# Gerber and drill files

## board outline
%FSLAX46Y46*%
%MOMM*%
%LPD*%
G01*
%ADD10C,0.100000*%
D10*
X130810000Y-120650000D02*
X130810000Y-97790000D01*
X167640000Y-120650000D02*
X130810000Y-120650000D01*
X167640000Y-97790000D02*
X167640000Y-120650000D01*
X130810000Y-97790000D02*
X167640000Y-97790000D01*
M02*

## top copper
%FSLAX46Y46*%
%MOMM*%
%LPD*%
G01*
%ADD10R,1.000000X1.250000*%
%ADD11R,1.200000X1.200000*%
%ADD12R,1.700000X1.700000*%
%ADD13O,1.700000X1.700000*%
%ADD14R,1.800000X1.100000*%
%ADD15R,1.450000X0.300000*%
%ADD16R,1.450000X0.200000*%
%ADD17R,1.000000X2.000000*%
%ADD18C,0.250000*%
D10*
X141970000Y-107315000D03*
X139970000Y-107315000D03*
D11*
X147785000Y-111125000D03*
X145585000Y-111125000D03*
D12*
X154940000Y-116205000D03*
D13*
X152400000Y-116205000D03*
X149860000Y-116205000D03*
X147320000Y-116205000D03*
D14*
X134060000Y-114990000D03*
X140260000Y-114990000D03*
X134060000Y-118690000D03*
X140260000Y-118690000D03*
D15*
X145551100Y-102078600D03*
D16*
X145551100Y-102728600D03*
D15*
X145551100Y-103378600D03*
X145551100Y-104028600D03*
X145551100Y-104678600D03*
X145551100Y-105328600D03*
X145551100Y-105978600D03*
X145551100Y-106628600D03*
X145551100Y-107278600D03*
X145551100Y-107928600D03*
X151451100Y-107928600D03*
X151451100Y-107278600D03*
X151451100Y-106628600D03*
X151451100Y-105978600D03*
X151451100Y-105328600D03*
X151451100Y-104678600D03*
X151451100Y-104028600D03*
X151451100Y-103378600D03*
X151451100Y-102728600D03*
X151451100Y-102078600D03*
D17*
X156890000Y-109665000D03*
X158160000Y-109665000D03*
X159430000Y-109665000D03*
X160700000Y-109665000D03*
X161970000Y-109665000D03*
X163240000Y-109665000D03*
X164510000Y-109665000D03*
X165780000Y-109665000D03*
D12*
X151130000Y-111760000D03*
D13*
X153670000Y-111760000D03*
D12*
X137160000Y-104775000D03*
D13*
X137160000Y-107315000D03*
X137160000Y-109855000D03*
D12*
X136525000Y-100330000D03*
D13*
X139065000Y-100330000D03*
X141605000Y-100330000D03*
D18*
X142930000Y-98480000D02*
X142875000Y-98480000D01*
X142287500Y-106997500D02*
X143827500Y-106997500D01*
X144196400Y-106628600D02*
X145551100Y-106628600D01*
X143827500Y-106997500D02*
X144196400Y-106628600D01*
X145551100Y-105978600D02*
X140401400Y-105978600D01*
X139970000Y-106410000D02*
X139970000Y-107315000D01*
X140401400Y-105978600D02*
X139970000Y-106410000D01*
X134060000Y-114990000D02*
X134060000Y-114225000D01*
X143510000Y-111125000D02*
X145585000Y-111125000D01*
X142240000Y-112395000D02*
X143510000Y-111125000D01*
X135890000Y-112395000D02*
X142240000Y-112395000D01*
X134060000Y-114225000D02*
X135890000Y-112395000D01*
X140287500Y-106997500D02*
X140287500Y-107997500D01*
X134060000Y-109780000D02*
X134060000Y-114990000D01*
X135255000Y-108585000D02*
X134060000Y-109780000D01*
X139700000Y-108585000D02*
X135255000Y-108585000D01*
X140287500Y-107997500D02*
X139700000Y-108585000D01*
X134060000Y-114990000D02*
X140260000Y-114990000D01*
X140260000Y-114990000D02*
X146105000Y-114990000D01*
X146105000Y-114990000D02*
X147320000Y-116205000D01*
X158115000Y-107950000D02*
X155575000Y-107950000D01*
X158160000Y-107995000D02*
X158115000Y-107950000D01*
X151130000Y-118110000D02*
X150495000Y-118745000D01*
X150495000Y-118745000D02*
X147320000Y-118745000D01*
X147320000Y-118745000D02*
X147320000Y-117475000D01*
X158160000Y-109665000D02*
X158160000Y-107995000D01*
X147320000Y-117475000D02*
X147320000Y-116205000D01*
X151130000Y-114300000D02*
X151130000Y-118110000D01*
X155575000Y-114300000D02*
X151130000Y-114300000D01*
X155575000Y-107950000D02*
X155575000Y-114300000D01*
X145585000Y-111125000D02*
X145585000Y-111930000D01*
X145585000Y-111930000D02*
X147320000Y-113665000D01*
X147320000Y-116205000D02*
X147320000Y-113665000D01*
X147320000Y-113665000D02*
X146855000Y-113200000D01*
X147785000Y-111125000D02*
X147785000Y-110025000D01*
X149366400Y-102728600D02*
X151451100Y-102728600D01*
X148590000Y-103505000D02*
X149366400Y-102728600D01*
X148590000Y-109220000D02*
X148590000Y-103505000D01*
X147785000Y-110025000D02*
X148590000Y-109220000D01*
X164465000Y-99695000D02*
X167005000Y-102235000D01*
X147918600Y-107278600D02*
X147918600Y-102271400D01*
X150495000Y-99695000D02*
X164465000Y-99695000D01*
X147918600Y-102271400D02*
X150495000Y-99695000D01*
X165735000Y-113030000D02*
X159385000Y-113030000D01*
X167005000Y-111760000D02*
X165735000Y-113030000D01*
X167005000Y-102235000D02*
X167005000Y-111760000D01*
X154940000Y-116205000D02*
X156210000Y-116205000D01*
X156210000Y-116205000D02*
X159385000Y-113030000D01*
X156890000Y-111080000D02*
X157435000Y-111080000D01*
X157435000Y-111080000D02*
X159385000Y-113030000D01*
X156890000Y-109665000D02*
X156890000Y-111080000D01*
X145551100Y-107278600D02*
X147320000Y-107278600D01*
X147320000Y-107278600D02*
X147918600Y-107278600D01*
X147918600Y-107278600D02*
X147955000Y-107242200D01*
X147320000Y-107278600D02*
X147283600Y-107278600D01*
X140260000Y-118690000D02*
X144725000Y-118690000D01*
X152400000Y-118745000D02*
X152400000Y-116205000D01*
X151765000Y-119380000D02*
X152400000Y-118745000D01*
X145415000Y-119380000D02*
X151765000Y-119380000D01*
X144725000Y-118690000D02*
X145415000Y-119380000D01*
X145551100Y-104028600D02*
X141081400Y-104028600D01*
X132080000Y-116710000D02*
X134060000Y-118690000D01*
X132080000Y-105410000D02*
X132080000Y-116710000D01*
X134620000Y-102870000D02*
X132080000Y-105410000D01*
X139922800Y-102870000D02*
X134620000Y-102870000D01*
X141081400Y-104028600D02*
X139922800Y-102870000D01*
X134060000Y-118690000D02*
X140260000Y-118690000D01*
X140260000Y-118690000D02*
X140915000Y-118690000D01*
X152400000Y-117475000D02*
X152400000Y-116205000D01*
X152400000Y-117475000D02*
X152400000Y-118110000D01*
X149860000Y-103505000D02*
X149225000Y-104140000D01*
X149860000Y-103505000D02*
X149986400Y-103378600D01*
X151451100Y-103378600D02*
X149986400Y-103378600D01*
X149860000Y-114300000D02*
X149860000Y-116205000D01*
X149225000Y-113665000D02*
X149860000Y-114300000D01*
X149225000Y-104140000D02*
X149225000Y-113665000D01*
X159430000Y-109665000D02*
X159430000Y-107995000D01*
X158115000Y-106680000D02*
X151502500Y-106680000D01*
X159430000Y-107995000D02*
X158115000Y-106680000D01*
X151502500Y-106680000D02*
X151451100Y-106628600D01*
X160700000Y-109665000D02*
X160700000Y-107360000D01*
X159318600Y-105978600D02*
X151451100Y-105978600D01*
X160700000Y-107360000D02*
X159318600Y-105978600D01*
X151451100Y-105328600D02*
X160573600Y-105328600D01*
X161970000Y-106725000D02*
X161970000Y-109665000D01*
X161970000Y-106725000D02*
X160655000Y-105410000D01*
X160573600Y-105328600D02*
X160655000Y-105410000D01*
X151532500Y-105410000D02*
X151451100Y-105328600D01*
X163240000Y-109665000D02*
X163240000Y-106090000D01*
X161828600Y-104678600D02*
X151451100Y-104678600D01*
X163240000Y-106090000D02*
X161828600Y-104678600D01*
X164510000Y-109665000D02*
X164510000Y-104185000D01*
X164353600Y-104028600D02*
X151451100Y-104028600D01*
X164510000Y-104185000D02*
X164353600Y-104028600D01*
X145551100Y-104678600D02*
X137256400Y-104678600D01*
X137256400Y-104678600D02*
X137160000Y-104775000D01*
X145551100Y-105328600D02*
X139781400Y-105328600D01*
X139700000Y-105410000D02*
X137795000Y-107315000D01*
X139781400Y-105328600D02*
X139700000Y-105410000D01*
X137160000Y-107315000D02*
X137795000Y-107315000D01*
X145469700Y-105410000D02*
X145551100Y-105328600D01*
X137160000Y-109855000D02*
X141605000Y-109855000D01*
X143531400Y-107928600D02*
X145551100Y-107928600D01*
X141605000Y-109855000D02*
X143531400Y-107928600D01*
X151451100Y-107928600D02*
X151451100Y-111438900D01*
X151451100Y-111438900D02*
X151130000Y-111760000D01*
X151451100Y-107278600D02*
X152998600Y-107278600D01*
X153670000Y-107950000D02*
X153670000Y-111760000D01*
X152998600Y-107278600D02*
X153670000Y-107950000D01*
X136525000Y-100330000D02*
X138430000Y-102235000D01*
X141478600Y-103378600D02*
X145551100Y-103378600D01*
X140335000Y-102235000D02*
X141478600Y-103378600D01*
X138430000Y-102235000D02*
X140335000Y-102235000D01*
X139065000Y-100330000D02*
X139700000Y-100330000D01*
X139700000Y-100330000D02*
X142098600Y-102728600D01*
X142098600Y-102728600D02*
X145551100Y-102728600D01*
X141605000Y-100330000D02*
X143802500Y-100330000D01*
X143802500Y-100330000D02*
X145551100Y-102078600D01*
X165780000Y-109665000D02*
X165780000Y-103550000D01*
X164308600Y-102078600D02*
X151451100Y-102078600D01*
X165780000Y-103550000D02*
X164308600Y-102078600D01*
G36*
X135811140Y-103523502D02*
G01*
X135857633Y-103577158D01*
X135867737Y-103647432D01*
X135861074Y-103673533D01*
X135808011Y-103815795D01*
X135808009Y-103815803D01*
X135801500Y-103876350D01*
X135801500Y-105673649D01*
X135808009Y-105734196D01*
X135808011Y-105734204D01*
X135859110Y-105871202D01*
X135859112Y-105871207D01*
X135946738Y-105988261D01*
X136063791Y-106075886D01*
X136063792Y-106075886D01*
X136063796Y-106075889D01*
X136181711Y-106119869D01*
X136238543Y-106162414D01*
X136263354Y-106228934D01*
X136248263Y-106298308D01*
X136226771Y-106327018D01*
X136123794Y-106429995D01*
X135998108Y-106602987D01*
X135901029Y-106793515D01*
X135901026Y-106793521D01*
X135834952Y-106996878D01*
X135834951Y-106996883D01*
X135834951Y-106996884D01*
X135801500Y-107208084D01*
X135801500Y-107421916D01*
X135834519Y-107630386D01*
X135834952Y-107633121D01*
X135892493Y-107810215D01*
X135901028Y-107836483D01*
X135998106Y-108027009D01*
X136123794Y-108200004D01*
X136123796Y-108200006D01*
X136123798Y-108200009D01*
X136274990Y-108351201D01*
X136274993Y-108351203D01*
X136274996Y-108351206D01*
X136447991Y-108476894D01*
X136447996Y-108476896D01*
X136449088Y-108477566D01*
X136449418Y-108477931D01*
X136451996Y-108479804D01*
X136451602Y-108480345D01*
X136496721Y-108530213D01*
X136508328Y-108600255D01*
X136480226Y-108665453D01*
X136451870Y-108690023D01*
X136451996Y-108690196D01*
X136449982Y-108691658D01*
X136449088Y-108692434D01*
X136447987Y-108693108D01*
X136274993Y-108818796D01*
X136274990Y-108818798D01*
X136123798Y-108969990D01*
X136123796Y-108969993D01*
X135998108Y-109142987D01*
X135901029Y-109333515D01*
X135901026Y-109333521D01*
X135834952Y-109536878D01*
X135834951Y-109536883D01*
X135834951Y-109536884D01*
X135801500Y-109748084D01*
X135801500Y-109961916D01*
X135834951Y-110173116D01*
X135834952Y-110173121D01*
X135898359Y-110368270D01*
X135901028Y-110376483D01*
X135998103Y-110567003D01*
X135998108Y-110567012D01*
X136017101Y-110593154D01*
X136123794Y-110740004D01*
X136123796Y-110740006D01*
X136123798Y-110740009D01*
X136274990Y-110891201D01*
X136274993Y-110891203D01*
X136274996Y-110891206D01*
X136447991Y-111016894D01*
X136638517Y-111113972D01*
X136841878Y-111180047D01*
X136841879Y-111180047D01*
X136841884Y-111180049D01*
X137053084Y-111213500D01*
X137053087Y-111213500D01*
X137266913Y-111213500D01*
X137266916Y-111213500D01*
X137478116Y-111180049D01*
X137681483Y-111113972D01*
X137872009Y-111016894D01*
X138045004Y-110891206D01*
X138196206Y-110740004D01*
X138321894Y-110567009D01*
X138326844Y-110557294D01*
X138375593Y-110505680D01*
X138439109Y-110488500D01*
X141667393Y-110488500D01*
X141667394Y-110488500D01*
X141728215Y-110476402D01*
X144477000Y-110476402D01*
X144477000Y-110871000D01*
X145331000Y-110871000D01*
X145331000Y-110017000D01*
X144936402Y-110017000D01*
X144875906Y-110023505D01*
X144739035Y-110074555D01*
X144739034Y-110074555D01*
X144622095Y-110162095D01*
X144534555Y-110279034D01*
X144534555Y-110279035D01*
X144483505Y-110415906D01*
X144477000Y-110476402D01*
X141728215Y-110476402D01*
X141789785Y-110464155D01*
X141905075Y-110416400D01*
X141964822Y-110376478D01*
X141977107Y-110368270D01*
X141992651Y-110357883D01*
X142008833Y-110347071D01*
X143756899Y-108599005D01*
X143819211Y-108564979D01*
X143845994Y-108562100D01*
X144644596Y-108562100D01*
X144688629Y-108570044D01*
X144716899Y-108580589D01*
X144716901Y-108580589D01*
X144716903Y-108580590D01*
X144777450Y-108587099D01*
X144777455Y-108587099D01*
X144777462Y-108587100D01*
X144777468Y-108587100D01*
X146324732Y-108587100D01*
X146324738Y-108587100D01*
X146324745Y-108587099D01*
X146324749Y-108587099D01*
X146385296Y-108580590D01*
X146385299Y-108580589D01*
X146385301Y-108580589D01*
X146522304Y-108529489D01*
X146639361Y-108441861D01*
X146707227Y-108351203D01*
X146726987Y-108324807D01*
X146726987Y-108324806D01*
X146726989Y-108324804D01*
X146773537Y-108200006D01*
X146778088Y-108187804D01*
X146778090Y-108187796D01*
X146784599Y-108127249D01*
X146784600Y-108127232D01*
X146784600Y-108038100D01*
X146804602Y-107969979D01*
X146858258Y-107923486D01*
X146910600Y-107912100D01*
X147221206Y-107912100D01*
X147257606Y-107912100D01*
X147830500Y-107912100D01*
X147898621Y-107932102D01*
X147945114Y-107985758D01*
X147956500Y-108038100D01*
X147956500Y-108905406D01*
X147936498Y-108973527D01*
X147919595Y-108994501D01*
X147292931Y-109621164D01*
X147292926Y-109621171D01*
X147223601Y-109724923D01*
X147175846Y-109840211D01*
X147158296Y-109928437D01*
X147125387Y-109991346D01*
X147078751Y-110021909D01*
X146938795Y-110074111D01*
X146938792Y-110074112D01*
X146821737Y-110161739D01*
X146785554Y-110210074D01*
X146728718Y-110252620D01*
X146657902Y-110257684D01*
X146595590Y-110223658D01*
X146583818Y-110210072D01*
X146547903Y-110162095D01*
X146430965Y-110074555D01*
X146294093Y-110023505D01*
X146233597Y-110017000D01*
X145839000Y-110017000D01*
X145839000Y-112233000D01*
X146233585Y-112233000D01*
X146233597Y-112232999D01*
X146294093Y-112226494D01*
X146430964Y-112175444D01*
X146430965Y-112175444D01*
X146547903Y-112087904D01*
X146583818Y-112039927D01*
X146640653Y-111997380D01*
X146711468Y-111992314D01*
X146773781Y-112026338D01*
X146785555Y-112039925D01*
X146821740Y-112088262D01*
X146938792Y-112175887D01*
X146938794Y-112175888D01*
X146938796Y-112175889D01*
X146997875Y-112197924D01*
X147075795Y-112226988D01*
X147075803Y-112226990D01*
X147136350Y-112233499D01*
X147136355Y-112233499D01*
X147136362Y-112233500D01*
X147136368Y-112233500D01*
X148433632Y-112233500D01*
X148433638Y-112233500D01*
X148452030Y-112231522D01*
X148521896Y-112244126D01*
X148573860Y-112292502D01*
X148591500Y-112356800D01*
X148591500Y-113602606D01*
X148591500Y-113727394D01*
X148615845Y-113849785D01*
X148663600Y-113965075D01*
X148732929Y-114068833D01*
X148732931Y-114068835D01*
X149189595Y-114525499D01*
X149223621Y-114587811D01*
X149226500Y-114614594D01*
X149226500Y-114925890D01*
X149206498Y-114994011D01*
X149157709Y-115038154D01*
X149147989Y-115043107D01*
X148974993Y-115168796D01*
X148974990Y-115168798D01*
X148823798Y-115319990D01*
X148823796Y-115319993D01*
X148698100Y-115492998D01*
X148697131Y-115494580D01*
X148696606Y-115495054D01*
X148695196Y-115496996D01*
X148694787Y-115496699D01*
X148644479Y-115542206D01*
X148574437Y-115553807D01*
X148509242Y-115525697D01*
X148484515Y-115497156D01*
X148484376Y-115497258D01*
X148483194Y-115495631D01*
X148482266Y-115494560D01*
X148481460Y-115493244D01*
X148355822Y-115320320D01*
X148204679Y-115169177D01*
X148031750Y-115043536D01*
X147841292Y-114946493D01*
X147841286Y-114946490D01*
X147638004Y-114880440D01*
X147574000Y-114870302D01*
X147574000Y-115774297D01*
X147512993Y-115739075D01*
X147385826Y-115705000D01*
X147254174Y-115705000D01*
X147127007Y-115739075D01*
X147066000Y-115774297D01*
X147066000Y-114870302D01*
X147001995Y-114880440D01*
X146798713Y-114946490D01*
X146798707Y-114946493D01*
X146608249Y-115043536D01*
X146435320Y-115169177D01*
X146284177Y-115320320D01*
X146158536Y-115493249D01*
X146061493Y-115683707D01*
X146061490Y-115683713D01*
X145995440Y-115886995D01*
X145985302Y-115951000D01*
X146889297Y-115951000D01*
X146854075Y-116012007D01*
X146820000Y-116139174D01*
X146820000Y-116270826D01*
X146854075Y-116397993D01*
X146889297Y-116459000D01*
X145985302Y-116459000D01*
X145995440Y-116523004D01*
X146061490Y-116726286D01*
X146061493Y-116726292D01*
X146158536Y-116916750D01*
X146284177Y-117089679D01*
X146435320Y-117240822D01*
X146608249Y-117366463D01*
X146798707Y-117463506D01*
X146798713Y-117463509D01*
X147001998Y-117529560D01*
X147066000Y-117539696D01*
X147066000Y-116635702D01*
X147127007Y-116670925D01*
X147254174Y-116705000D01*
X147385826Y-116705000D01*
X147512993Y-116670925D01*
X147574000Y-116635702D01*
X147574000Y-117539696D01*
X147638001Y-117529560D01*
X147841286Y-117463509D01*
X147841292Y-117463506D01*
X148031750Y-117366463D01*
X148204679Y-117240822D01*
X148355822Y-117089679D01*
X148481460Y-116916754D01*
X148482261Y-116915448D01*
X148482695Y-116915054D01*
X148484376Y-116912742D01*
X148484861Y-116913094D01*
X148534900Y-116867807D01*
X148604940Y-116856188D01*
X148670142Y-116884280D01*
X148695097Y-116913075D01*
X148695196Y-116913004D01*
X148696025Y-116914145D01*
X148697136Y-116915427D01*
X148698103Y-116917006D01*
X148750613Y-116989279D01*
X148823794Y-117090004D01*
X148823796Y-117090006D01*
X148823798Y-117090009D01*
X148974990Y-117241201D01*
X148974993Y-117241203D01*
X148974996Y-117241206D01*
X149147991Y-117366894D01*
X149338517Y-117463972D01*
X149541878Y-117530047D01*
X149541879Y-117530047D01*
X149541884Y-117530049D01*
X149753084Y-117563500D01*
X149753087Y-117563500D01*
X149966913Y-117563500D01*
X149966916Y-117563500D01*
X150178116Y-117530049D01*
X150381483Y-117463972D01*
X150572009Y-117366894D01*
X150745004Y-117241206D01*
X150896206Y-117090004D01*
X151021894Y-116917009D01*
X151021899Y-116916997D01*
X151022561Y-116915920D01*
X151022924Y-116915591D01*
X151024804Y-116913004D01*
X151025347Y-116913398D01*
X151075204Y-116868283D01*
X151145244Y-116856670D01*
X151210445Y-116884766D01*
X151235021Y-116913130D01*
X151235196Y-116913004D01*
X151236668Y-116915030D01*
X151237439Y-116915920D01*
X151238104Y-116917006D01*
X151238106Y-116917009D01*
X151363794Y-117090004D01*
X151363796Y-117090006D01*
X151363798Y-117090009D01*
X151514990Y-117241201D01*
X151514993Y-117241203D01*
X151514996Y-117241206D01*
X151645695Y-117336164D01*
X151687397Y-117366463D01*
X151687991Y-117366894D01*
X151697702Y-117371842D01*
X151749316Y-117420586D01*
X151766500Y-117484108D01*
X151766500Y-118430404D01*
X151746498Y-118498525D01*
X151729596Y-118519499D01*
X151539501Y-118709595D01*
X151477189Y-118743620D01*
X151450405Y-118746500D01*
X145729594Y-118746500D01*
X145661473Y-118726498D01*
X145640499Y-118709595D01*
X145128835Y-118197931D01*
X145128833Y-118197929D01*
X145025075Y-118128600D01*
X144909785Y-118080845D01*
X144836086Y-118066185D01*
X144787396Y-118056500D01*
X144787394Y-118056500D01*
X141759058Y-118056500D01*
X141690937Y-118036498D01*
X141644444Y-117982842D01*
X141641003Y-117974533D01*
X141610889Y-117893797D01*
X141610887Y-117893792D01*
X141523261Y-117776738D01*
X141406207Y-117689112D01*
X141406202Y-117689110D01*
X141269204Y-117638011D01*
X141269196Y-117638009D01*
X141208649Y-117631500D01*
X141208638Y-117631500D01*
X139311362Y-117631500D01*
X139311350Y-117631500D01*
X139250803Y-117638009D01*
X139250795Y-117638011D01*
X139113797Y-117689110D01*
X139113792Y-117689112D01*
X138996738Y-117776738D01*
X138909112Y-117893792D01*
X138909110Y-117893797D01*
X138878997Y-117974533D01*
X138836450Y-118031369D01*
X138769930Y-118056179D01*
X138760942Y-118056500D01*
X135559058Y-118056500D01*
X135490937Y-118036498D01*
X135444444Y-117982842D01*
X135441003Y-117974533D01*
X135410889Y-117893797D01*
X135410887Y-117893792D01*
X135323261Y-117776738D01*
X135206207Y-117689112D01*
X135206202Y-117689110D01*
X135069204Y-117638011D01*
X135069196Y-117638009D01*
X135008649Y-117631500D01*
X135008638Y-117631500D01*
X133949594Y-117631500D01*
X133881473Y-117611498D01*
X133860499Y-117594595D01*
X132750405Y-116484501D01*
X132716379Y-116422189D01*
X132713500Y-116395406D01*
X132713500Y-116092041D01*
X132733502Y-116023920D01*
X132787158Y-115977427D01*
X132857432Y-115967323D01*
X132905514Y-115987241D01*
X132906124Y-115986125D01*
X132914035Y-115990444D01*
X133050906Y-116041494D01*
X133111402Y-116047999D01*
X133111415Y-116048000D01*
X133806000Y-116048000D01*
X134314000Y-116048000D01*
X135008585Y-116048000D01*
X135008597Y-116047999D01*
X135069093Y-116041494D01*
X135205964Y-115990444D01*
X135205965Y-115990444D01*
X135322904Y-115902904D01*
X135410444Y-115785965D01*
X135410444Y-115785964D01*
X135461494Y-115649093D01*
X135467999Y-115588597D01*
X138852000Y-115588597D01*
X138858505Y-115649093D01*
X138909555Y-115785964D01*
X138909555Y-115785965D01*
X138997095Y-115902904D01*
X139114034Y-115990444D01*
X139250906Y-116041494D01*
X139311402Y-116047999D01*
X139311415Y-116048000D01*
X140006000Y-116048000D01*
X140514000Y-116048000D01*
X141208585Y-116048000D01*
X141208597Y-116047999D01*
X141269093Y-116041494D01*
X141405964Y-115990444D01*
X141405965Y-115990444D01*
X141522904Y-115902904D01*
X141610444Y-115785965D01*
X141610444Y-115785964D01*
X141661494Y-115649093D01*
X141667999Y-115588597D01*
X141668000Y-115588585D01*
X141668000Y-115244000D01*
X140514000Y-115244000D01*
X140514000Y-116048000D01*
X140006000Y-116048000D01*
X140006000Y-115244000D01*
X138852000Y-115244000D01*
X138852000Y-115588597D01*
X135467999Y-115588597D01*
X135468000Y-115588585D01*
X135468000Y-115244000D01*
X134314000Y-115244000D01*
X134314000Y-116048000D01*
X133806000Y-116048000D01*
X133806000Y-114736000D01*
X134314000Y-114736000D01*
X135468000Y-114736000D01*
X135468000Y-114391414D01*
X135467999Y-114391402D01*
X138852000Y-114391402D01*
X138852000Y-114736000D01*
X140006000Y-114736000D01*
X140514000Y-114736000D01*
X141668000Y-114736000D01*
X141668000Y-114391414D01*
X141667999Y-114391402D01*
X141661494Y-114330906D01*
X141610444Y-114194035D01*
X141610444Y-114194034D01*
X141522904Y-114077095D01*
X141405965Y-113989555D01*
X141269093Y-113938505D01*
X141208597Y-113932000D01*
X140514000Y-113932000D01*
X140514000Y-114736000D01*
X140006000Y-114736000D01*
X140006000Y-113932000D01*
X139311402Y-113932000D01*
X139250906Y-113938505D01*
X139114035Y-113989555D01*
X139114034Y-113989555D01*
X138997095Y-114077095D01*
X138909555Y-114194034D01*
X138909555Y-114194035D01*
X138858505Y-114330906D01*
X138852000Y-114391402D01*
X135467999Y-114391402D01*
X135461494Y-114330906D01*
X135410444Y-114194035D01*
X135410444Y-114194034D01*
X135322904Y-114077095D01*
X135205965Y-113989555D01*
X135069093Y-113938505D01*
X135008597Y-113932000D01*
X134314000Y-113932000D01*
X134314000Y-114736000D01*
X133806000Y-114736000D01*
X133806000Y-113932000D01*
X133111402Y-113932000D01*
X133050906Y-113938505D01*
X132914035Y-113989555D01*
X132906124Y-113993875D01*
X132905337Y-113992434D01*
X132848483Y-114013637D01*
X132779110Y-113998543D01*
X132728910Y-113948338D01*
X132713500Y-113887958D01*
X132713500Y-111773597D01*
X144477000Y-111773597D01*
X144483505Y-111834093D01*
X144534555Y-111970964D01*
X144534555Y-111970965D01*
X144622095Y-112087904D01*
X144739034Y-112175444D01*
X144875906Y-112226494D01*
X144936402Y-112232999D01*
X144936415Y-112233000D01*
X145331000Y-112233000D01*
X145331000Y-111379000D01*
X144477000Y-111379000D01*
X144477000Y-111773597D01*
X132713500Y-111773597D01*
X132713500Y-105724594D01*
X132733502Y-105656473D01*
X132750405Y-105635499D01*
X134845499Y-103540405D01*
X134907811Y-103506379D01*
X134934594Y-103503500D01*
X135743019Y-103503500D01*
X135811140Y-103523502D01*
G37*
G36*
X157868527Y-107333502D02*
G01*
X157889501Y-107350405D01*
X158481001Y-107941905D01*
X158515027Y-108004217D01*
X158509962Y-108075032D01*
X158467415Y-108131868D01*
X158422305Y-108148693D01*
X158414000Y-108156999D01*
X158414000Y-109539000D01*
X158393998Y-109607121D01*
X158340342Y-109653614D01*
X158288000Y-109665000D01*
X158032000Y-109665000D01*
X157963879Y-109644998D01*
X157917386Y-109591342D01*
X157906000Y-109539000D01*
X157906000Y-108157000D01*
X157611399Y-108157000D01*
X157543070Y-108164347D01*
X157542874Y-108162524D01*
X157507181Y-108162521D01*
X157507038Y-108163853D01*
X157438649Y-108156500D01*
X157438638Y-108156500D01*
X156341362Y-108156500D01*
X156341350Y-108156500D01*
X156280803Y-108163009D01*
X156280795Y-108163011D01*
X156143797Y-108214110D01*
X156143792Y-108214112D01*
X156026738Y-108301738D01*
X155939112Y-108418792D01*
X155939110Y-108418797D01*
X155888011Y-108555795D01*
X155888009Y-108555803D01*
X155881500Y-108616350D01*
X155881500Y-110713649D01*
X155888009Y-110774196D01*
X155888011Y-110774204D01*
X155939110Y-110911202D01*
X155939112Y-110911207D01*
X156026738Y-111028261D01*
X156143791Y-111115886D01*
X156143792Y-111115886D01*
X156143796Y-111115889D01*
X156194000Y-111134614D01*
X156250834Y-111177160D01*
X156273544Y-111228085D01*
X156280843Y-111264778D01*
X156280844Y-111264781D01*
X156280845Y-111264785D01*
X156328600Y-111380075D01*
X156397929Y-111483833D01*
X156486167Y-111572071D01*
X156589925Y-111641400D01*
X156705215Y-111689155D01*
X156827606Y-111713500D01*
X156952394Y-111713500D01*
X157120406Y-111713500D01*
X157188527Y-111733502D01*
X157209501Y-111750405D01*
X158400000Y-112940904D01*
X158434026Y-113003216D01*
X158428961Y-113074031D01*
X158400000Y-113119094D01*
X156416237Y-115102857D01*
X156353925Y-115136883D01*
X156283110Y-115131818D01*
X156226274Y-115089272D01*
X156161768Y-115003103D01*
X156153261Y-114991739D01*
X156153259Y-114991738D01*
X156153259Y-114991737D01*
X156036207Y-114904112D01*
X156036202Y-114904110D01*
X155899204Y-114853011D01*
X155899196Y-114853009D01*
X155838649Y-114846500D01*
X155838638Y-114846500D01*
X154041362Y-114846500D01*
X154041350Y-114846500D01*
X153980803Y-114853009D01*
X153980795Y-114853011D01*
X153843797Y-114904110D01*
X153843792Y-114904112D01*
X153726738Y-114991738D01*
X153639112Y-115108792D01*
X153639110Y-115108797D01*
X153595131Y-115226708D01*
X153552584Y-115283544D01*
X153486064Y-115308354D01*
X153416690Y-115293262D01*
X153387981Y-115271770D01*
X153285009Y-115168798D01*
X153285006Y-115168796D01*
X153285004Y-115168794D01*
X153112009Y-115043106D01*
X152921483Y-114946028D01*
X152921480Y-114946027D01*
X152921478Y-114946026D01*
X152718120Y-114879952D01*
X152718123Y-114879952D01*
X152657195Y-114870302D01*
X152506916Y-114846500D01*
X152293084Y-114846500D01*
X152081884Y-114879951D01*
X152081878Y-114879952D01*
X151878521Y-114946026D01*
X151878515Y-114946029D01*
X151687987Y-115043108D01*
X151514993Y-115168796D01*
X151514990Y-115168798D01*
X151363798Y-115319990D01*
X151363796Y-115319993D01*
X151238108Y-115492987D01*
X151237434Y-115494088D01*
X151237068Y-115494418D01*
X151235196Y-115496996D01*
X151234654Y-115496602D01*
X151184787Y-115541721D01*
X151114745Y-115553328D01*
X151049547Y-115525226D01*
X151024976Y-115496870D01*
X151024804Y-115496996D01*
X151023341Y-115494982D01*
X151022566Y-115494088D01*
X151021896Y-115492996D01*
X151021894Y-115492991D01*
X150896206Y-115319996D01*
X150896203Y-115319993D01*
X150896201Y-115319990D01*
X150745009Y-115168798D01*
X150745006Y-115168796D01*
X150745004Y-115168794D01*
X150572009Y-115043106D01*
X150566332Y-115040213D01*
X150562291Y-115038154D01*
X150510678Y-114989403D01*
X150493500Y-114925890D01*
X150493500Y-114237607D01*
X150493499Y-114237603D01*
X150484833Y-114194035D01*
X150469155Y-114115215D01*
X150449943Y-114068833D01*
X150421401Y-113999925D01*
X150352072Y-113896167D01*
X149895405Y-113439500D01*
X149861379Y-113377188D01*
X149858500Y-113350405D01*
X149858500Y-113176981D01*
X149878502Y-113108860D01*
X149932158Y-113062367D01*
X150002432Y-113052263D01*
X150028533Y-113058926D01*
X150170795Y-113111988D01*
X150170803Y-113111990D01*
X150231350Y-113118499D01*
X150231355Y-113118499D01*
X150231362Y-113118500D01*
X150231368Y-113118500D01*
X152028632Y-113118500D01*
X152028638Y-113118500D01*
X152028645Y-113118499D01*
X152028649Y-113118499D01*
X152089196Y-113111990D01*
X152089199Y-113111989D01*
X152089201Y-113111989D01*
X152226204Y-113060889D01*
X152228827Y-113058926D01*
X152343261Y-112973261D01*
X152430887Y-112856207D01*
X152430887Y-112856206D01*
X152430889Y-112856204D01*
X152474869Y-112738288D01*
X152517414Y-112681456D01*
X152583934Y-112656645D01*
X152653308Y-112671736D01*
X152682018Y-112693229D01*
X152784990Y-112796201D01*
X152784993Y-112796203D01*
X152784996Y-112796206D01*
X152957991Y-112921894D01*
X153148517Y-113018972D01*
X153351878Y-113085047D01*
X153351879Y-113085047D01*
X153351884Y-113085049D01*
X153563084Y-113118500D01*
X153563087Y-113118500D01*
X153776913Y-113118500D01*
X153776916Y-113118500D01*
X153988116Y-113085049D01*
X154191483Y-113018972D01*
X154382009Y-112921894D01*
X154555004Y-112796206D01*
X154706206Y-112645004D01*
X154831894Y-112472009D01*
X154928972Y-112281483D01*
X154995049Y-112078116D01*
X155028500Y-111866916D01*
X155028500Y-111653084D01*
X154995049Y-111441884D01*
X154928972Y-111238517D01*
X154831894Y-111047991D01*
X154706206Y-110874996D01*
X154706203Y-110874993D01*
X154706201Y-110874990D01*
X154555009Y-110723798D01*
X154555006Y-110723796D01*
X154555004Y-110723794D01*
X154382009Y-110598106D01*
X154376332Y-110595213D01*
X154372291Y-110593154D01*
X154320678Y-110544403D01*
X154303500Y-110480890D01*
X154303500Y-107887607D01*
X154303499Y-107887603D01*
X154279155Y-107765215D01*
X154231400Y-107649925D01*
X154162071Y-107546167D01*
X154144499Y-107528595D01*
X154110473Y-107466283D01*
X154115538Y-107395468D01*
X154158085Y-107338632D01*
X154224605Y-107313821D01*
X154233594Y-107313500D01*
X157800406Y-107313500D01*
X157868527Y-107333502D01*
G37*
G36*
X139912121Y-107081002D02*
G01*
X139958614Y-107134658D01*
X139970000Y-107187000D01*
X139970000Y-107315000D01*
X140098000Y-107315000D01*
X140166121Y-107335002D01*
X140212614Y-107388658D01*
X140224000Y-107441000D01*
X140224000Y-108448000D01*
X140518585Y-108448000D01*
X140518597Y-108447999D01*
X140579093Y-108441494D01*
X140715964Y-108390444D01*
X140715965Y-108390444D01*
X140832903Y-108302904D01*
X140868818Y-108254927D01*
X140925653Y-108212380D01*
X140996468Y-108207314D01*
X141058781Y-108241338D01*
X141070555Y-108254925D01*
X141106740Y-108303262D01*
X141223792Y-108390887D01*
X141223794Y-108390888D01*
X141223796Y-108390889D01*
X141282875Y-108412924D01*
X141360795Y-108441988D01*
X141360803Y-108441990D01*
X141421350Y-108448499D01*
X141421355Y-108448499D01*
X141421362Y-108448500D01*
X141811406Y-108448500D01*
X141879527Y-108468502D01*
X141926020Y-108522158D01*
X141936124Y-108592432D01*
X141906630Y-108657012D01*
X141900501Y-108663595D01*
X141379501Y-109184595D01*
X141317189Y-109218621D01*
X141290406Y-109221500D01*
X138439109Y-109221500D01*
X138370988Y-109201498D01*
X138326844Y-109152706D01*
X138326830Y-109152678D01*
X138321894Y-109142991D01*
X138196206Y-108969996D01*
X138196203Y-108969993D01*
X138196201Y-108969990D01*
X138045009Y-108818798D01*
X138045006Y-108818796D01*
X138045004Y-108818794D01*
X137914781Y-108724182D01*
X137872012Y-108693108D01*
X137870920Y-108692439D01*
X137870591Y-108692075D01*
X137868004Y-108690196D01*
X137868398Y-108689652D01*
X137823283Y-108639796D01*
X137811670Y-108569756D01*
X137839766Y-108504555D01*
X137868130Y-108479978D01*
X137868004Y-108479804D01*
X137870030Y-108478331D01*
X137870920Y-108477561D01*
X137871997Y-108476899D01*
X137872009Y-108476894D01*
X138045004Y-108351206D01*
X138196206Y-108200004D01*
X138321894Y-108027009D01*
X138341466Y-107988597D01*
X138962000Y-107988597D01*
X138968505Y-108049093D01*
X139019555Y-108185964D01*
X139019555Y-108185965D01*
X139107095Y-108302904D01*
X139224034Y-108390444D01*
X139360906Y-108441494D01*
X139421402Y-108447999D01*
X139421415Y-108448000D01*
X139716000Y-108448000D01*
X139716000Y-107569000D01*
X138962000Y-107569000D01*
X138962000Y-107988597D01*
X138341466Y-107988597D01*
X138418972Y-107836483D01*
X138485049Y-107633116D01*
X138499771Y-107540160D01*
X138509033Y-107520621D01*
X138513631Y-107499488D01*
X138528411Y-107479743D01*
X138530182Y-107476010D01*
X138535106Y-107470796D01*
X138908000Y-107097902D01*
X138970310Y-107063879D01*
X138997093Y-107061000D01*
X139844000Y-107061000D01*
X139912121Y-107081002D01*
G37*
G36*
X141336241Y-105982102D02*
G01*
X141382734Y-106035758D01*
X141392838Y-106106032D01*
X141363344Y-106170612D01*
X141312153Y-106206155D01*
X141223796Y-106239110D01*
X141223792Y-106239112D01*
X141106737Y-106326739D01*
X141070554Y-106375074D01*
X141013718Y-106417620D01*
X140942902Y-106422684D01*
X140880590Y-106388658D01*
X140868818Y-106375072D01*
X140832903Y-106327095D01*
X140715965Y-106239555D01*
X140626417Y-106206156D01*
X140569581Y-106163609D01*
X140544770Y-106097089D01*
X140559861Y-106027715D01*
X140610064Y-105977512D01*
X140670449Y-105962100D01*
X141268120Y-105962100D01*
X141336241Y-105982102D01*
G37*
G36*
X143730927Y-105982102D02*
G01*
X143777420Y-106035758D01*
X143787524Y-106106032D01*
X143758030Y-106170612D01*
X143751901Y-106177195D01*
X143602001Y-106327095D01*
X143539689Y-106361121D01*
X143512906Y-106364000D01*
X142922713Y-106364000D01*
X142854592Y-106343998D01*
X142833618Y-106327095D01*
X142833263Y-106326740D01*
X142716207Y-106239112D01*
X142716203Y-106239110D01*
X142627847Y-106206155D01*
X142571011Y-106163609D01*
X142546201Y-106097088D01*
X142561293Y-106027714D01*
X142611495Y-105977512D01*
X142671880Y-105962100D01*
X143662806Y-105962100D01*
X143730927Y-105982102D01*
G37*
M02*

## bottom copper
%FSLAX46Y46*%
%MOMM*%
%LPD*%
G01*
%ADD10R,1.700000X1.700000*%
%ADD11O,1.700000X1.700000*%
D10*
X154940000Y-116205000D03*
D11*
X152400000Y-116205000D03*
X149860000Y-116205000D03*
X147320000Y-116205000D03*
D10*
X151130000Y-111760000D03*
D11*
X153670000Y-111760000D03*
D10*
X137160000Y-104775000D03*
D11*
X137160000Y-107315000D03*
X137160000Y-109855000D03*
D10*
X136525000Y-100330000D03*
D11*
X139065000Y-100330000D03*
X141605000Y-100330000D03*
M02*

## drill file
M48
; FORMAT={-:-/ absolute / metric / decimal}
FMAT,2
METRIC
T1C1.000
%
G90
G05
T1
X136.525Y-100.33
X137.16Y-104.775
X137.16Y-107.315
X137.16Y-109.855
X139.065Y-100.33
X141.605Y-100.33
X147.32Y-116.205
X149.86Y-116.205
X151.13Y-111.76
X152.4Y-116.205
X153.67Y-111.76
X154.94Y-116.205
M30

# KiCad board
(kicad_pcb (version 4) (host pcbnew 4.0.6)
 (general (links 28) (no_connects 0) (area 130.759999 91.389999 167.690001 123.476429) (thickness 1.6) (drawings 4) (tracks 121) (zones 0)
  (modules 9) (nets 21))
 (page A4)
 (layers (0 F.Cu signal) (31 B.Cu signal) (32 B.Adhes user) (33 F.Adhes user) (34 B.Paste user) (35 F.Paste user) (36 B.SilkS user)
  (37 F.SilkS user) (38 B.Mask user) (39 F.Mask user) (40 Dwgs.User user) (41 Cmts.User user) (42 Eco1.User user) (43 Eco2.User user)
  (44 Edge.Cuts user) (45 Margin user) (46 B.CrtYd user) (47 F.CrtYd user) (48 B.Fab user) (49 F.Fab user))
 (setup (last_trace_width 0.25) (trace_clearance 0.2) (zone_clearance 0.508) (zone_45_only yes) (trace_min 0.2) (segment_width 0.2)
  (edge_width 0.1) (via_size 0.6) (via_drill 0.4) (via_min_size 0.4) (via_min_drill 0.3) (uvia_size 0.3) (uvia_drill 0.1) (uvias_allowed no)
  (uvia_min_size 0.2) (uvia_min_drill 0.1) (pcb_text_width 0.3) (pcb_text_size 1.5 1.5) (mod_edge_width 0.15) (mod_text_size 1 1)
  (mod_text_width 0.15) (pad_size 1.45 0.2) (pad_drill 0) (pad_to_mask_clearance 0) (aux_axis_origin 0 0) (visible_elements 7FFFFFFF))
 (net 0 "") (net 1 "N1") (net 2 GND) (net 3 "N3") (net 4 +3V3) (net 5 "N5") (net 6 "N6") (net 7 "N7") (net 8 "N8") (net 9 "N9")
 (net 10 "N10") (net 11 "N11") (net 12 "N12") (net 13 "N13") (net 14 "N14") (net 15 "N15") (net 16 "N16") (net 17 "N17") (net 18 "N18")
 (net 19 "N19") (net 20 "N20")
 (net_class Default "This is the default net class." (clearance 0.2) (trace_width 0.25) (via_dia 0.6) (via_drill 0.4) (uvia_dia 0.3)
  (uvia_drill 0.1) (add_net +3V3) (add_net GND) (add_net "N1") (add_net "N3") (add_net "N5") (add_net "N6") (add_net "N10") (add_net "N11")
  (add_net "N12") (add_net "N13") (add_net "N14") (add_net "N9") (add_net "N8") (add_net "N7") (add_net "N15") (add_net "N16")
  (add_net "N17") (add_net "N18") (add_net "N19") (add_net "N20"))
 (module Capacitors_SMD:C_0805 (layer F.Cu) (at 140.97 107.315 180)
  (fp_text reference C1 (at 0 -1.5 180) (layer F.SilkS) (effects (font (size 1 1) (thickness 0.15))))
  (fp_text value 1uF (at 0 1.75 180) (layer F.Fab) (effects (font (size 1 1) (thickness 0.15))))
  (pad 1 smd rect (at -1 0 180) (size 1 1.25) (layers F.Cu F.Paste F.Mask) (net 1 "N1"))
  (pad 2 smd rect (at 1 0 180) (size 1 1.25) (layers F.Cu F.Paste F.Mask) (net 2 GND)))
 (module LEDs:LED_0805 (layer F.Cu) (at 146.685 111.125)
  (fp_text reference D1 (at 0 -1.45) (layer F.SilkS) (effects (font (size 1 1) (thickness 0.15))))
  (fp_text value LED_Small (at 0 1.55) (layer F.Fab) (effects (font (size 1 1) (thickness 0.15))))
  (pad 2 smd rect (at 1.1 0 180) (size 1.2 1.2) (layers F.Cu F.Paste F.Mask) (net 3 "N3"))
  (pad 1 smd rect (at -1.1 0 180) (size 1.2 1.2) (layers F.Cu F.Paste F.Mask) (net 2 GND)))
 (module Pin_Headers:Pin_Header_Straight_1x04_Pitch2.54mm (layer F.Cu) (at 154.94 116.205 270)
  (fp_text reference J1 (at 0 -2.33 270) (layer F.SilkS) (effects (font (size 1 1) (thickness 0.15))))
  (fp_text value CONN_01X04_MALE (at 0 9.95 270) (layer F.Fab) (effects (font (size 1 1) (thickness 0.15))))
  (pad 1 thru_hole rect (at 0 0 270) (size 1.7 1.7) (drill 1) (layers *.Cu *.Mask) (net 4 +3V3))
  (pad 2 thru_hole oval (at 0 2.54 270) (size 1.7 1.7) (drill 1) (layers *.Cu *.Mask) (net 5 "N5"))
  (pad 3 thru_hole oval (at 0 5.08 270) (size 1.7 1.7) (drill 1) (layers *.Cu *.Mask) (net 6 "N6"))
  (pad 4 thru_hole oval (at 0 7.62 270) (size 1.7 1.7) (drill 1) (layers *.Cu *.Mask) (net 2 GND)))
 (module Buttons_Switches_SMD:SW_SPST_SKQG (layer F.Cu) (at 137.16 116.84)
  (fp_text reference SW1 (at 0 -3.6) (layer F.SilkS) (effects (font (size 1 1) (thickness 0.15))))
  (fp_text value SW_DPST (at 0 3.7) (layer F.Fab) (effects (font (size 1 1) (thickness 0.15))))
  (pad 1 smd rect (at -3.1 -1.85) (size 1.8 1.1) (layers F.Cu F.Paste F.Mask) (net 2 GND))
  (pad 1 smd rect (at 3.1 -1.85) (size 1.8 1.1) (layers F.Cu F.Paste F.Mask) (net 2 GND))
  (pad 2 smd rect (at -3.1 1.85) (size 1.8 1.1) (layers F.Cu F.Paste F.Mask) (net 5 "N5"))
  (pad 2 smd rect (at 3.1 1.85) (size 1.8 1.1) (layers F.Cu F.Paste F.Mask) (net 5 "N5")))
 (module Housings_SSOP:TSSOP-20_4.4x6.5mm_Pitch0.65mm (layer F.Cu) (at 148.5011 105.0036)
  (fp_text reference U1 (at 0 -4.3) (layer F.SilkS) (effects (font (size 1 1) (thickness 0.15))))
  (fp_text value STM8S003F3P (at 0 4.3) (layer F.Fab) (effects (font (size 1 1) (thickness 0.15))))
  (pad 1 smd rect (at -2.95 -2.925) (size 1.45 0.3) (layers F.Cu F.Paste F.Mask) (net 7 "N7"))
  (pad 2 smd rect (at -2.95 -2.275) (size 1.45 0.2) (layers F.Cu F.Paste F.Mask) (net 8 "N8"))
  (pad 3 smd rect (at -2.95 -1.625) (size 1.45 0.3) (layers F.Cu F.Paste F.Mask) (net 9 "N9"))
  (pad 4 smd rect (at -2.95 -0.975) (size 1.45 0.3) (layers F.Cu F.Paste F.Mask) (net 5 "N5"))
  (pad 5 smd rect (at -2.95 -0.325) (size 1.45 0.3) (layers F.Cu F.Paste F.Mask) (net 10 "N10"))
  (pad 6 smd rect (at -2.95 0.325) (size 1.45 0.3) (layers F.Cu F.Paste F.Mask) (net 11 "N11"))
  (pad 7 smd rect (at -2.95 0.975) (size 1.45 0.3) (layers F.Cu F.Paste F.Mask) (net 2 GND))
  (pad 8 smd rect (at -2.95 1.625) (size 1.45 0.3) (layers F.Cu F.Paste F.Mask) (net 1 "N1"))
  (pad 9 smd rect (at -2.95 2.275) (size 1.45 0.3) (layers F.Cu F.Paste F.Mask) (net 4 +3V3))
  (pad 10 smd rect (at -2.95 2.925) (size 1.45 0.3) (layers F.Cu F.Paste F.Mask) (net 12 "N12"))
  (pad 11 smd rect (at 2.95 2.925) (size 1.45 0.3) (layers F.Cu F.Paste F.Mask) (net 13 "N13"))
  (pad 12 smd rect (at 2.95 2.275) (size 1.45 0.3) (layers F.Cu F.Paste F.Mask) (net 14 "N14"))
  (pad 13 smd rect (at 2.95 1.625) (size 1.45 0.3) (layers F.Cu F.Paste F.Mask) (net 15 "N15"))
  (pad 14 smd rect (at 2.95 0.975) (size 1.45 0.3) (layers F.Cu F.Paste F.Mask) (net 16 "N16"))
  (pad 15 smd rect (at 2.95 0.325) (size 1.45 0.3) (layers F.Cu F.Paste F.Mask) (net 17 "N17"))
  (pad 16 smd rect (at 2.95 -0.325) (size 1.45 0.3) (layers F.Cu F.Paste F.Mask) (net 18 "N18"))
  (pad 17 smd rect (at 2.95 -0.975) (size 1.45 0.3) (layers F.Cu F.Paste F.Mask) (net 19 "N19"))
  (pad 18 smd rect (at 2.95 -1.625) (size 1.45 0.3) (layers F.Cu F.Paste F.Mask) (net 6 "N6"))
  (pad 19 smd rect (at 2.95 -2.275) (size 1.45 0.3) (layers F.Cu F.Paste F.Mask) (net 3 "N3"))
  (pad 20 smd rect (at 2.95 -2.925) (size 1.45 0.3) (layers F.Cu F.Paste F.Mask) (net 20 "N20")))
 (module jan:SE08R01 (layer F.Cu) (at 161.29 100.965)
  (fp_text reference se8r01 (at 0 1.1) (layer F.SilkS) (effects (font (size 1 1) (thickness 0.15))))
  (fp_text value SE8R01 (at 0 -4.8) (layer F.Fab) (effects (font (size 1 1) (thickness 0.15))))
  (pad 1 smd rect (at -4.4 8.7) (size 1 2) (layers F.Cu F.Paste F.Mask) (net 4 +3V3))
  (pad 2 smd rect (at -3.13 8.7) (size 1 2) (layers F.Cu F.Paste F.Mask) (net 2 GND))
  (pad 3 smd rect (at -1.86 8.7) (size 1 2) (layers F.Cu F.Paste F.Mask) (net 15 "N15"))
  (pad 4 smd rect (at -0.59 8.7) (size 1 2) (layers F.Cu F.Paste F.Mask) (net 16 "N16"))
  (pad 5 smd rect (at 0.68 8.7) (size 1 2) (layers F.Cu F.Paste F.Mask) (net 17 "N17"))
  (pad 6 smd rect (at 1.95 8.7) (size 1 2) (layers F.Cu F.Paste F.Mask) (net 18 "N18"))
  (pad 7 smd rect (at 3.22 8.7) (size 1 2) (layers F.Cu F.Paste F.Mask) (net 19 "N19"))
  (pad 8 smd rect (at 4.49 8.7) (size 1 2) (layers F.Cu F.Paste F.Mask) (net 20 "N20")))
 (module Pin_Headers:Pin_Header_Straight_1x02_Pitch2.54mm (layer F.Cu) (at 151.13 111.76 90)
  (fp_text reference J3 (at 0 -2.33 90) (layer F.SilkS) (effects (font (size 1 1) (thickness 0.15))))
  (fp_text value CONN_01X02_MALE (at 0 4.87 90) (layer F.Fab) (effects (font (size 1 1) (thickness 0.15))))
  (pad 1 thru_hole rect (at 0 0 90) (size 1.7 1.7) (drill 1) (layers *.Cu *.Mask) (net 13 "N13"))
  (pad 2 thru_hole oval (at 0 2.54 90) (size 1.7 1.7) (drill 1) (layers *.Cu *.Mask) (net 14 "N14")))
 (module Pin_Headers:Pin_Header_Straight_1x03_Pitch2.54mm (layer F.Cu) (at 137.16 104.775)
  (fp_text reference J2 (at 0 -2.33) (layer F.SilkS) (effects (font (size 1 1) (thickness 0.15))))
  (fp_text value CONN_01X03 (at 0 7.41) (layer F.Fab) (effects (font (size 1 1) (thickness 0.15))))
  (pad 1 thru_hole rect (at 0 0) (size 1.7 1.7) (drill 1) (layers *.Cu *.Mask) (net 10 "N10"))
  (pad 2 thru_hole oval (at 0 2.54) (size 1.7 1.7) (drill 1) (layers *.Cu *.Mask) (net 11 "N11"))
  (pad 3 thru_hole oval (at 0 5.08) (size 1.7 1.7) (drill 1) (layers *.Cu *.Mask) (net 12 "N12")))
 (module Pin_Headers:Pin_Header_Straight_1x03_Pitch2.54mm (layer F.Cu) (at 136.525 100.33 90)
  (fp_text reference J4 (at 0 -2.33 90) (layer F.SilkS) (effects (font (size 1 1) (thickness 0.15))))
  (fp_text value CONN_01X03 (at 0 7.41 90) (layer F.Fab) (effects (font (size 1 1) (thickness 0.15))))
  (pad 1 thru_hole rect (at 0 0 90) (size 1.7 1.7) (drill 1) (layers *.Cu *.Mask) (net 9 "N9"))
  (pad 2 thru_hole oval (at 0 2.54 90) (size 1.7 1.7) (drill 1) (layers *.Cu *.Mask) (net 8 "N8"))
  (pad 3 thru_hole oval (at 0 5.08 90) (size 1.7 1.7) (drill 1) (layers *.Cu *.Mask) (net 7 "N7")))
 (gr_line (start 130.81 120.65) (end 130.81 97.79) (angle 90) (layer Edge.Cuts) (width 0.1))
 (gr_line (start 167.64 120.65) (end 130.81 120.65) (angle 90) (layer Edge.Cuts) (width 0.1))
 (gr_line (start 167.64 97.79) (end 167.64 120.65) (angle 90) (layer Edge.Cuts) (width 0.1))
 (gr_line (start 130.81 97.79) (end 167.64 97.79) (angle 90) (layer Edge.Cuts) (width 0.1))
 (segment (start 142.93 98.48) (end 142.875 98.48) (width 0.25) (layer F.Cu) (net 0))
 (segment (start 142.2875 106.9975) (end 143.8275 106.9975) (width 0.25) (layer F.Cu) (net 1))
 (segment (start 144.1964 106.6286) (end 145.5511 106.6286) (width 0.25) (layer F.Cu) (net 1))
 (segment (start 143.8275 106.9975) (end 144.1964 106.6286) (width 0.25) (layer F.Cu) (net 1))
 (segment (start 145.5511 105.9786) (end 140.4014 105.9786) (width 0.25) (layer F.Cu) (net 2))
 (segment (start 139.97 106.41) (end 139.97 107.315) (width 0.25) (layer F.Cu) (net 2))
 (segment (start 140.4014 105.9786) (end 139.97 106.41) (width 0.25) (layer F.Cu) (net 2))
 (segment (start 134.06 114.99) (end 134.06 114.225) (width 0.25) (layer F.Cu) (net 2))
 (segment (start 143.51 111.125) (end 145.585 111.125) (width 0.25) (layer F.Cu) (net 2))
 (segment (start 142.24 112.395) (end 143.51 111.125) (width 0.25) (layer F.Cu) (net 2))
 (segment (start 135.89 112.395) (end 142.24 112.395) (width 0.25) (layer F.Cu) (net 2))
 (segment (start 134.06 114.225) (end 135.89 112.395) (width 0.25) (layer F.Cu) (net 2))
 (segment (start 140.2875 106.9975) (end 140.2875 107.9975) (width 0.25) (layer F.Cu) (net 2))
 (segment (start 134.06 109.78) (end 134.06 114.99) (width 0.25) (layer F.Cu) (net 2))
 (segment (start 135.255 108.585) (end 134.06 109.78) (width 0.25) (layer F.Cu) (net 2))
 (segment (start 139.7 108.585) (end 135.255 108.585) (width 0.25) (layer F.Cu) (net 2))
 (segment (start 140.2875 107.9975) (end 139.7 108.585) (width 0.25) (layer F.Cu) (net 2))
 (segment (start 134.06 114.99) (end 140.26 114.99) (width 0.25) (layer F.Cu) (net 2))
 (segment (start 140.26 114.99) (end 146.105 114.99) (width 0.25) (layer F.Cu) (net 2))
 (segment (start 146.105 114.99) (end 147.32 116.205) (width 0.25) (layer F.Cu) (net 2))
 (segment (start 158.115 107.95) (end 155.575 107.95) (width 0.25) (layer F.Cu) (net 2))
 (segment (start 158.16 107.995) (end 158.115 107.95) (width 0.25) (layer F.Cu) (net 2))
 (segment (start 151.13 118.11) (end 150.495 118.745) (width 0.25) (layer F.Cu) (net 2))
 (segment (start 150.495 118.745) (end 147.32 118.745) (width 0.25) (layer F.Cu) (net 2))
 (segment (start 147.32 118.745) (end 147.32 117.475) (width 0.25) (layer F.Cu) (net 2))
 (segment (start 158.16 109.665) (end 158.16 107.995) (width 0.25) (layer F.Cu) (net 2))
 (segment (start 147.32 117.475) (end 147.32 116.205) (width 0.25) (layer F.Cu) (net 2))
 (segment (start 151.13 114.3) (end 151.13 118.11) (width 0.25) (layer F.Cu) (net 2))
 (segment (start 155.575 114.3) (end 151.13 114.3) (width 0.25) (layer F.Cu) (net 2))
 (segment (start 155.575 107.95) (end 155.575 114.3) (width 0.25) (layer F.Cu) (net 2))
 (segment (start 145.585 111.125) (end 145.585 111.93) (width 0.25) (layer F.Cu) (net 2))
 (segment (start 145.585 111.93) (end 147.32 113.665) (width 0.25) (layer F.Cu) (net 2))
 (segment (start 147.32 116.205) (end 147.32 113.665) (width 0.25) (layer F.Cu) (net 2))
 (segment (start 147.32 113.665) (end 146.855 113.2) (width 0.25) (layer F.Cu) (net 2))
 (segment (start 147.785 111.125) (end 147.785 110.025) (width 0.25) (layer F.Cu) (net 3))
 (segment (start 149.3664 102.7286) (end 151.4511 102.7286) (width 0.25) (layer F.Cu) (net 3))
 (segment (start 148.59 103.505) (end 149.3664 102.7286) (width 0.25) (layer F.Cu) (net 3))
 (segment (start 148.59 109.22) (end 148.59 103.505) (width 0.25) (layer F.Cu) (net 3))
 (segment (start 147.785 110.025) (end 148.59 109.22) (width 0.25) (layer F.Cu) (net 3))
 (segment (start 164.465 99.695) (end 167.005 102.235) (width 0.25) (layer F.Cu) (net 4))
 (segment (start 147.9186 107.2786) (end 147.9186 102.2714) (width 0.25) (layer F.Cu) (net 4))
 (segment (start 150.495 99.695) (end 164.465 99.695) (width 0.25) (layer F.Cu) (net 4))
 (segment (start 147.9186 102.2714) (end 150.495 99.695) (width 0.25) (layer F.Cu) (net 4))
 (segment (start 165.735 113.03) (end 159.385 113.03) (width 0.25) (layer F.Cu) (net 4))
 (segment (start 167.005 111.76) (end 165.735 113.03) (width 0.25) (layer F.Cu) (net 4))
 (segment (start 167.005 102.235) (end 167.005 111.76) (width 0.25) (layer F.Cu) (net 4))
 (segment (start 154.94 116.205) (end 156.21 116.205) (width 0.25) (layer F.Cu) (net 4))
 (segment (start 156.21 116.205) (end 159.385 113.03) (width 0.25) (layer F.Cu) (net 4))
 (segment (start 156.89 111.08) (end 157.435 111.08) (width 0.25) (layer F.Cu) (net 4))
 (segment (start 157.435 111.08) (end 159.385 113.03) (width 0.25) (layer F.Cu) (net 4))
 (segment (start 156.89 109.665) (end 156.89 111.08) (width 0.25) (layer F.Cu) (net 4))
 (segment (start 145.5511 107.2786) (end 147.32 107.2786) (width 0.25) (layer F.Cu) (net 4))
 (segment (start 147.32 107.2786) (end 147.9186 107.2786) (width 0.25) (layer F.Cu) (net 4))
 (segment (start 147.9186 107.2786) (end 147.955 107.2422) (width 0.25) (layer F.Cu) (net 4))
 (segment (start 147.32 107.2786) (end 147.2836 107.2786) (width 0.25) (layer F.Cu) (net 4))
 (segment (start 140.26 118.69) (end 144.725 118.69) (width 0.25) (layer F.Cu) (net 5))
 (segment (start 152.4 118.745) (end 152.4 116.205) (width 0.25) (layer F.Cu) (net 5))
 (segment (start 151.765 119.38) (end 152.4 118.745) (width 0.25) (layer F.Cu) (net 5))
 (segment (start 145.415 119.38) (end 151.765 119.38) (width 0.25) (layer F.Cu) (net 5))
 (segment (start 144.725 118.69) (end 145.415 119.38) (width 0.25) (layer F.Cu) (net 5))
 (segment (start 145.5511 104.0286) (end 141.0814 104.0286) (width 0.25) (layer F.Cu) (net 5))
 (segment (start 132.08 116.71) (end 134.06 118.69) (width 0.25) (layer F.Cu) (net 5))
 (segment (start 132.08 105.41) (end 132.08 116.71) (width 0.25) (layer F.Cu) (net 5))
 (segment (start 134.62 102.87) (end 132.08 105.41) (width 0.25) (layer F.Cu) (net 5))
 (segment (start 139.9228 102.87) (end 134.62 102.87) (width 0.25) (layer F.Cu) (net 5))
 (segment (start 141.0814 104.0286) (end 139.9228 102.87) (width 0.25) (layer F.Cu) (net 5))
 (segment (start 134.06 118.69) (end 140.26 118.69) (width 0.25) (layer F.Cu) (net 5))
 (segment (start 140.26 118.69) (end 140.915 118.69) (width 0.25) (layer F.Cu) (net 5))
 (segment (start 152.4 117.475) (end 152.4 116.205) (width 0.25) (layer F.Cu) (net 5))
 (segment (start 152.4 117.475) (end 152.4 118.11) (width 0.25) (layer F.Cu) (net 5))
 (segment (start 149.86 103.505) (end 149.225 104.14) (width 0.25) (layer F.Cu) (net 6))
 (segment (start 149.86 103.505) (end 149.9864 103.3786) (width 0.25) (layer F.Cu) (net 6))
 (segment (start 151.4511 103.3786) (end 149.9864 103.3786) (width 0.25) (layer F.Cu) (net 6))
 (segment (start 149.86 114.3) (end 149.86 116.205) (width 0.25) (layer F.Cu) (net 6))
 (segment (start 149.225 113.665) (end 149.86 114.3) (width 0.25) (layer F.Cu) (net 6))
 (segment (start 149.225 104.14) (end 149.225 113.665) (width 0.25) (layer F.Cu) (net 6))
 (segment (start 159.43 109.665) (end 159.43 107.995) (width 0.25) (layer F.Cu) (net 15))
 (segment (start 158.115 106.68) (end 151.5025 106.68) (width 0.25) (layer F.Cu) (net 15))
 (segment (start 159.43 107.995) (end 158.115 106.68) (width 0.25) (layer F.Cu) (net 15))
 (segment (start 151.5025 106.68) (end 151.4511 106.6286) (width 0.25) (layer F.Cu) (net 15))
 (segment (start 160.7 109.665) (end 160.7 107.36) (width 0.25) (layer F.Cu) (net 16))
 (segment (start 159.3186 105.9786) (end 151.4511 105.9786) (width 0.25) (layer F.Cu) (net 16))
 (segment (start 160.7 107.36) (end 159.3186 105.9786) (width 0.25) (layer F.Cu) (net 16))
 (segment (start 151.4511 105.3286) (end 160.5736 105.3286) (width 0.25) (layer F.Cu) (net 17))
 (segment (start 161.97 106.725) (end 161.97 109.665) (width 0.25) (layer F.Cu) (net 17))
 (segment (start 161.97 106.725) (end 160.655 105.41) (width 0.25) (layer F.Cu) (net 17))
 (segment (start 160.5736 105.3286) (end 160.655 105.41) (width 0.25) (layer F.Cu) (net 17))
 (segment (start 151.5325 105.41) (end 151.4511 105.3286) (width 0.25) (layer F.Cu) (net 17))
 (segment (start 163.24 109.665) (end 163.24 106.09) (width 0.25) (layer F.Cu) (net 18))
 (segment (start 161.8286 104.6786) (end 151.4511 104.6786) (width 0.25) (layer F.Cu) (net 18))
 (segment (start 163.24 106.09) (end 161.8286 104.6786) (width 0.25) (layer F.Cu) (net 18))
 (segment (start 164.51 109.665) (end 164.51 104.185) (width 0.25) (layer F.Cu) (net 19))
 (segment (start 164.3536 104.0286) (end 151.4511 104.0286) (width 0.25) (layer F.Cu) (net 19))
 (segment (start 164.51 104.185) (end 164.3536 104.0286) (width 0.25) (layer F.Cu) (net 19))
 (segment (start 145.5511 104.6786) (end 137.2564 104.6786) (width 0.25) (layer F.Cu) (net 10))
 (segment (start 137.2564 104.6786) (end 137.16 104.775) (width 0.25) (layer F.Cu) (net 10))
 (segment (start 145.5511 105.3286) (end 139.7814 105.3286) (width 0.25) (layer F.Cu) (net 11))
 (segment (start 139.7 105.41) (end 137.795 107.315) (width 0.25) (layer F.Cu) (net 11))
 (segment (start 139.7814 105.3286) (end 139.7 105.41) (width 0.25) (layer F.Cu) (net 11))
 (segment (start 137.16 107.315) (end 137.795 107.315) (width 0.25) (layer F.Cu) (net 11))
 (segment (start 145.4697 105.41) (end 145.5511 105.3286) (width 0.25) (layer F.Cu) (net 11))
 (segment (start 137.16 109.855) (end 141.605 109.855) (width 0.25) (layer F.Cu) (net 12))
 (segment (start 143.5314 107.9286) (end 145.5511 107.9286) (width 0.25) (layer F.Cu) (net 12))
 (segment (start 141.605 109.855) (end 143.5314 107.9286) (width 0.25) (layer F.Cu) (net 12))
 (segment (start 151.4511 107.9286) (end 151.4511 111.4389) (width 0.25) (layer F.Cu) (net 13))
 (segment (start 151.4511 111.4389) (end 151.13 111.76) (width 0.25) (layer F.Cu) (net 13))
 (segment (start 151.4511 107.2786) (end 152.9986 107.2786) (width 0.25) (layer F.Cu) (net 14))
 (segment (start 153.67 107.95) (end 153.67 111.76) (width 0.25) (layer F.Cu) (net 14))
 (segment (start 152.9986 107.2786) (end 153.67 107.95) (width 0.25) (layer F.Cu) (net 14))
 (segment (start 136.525 100.33) (end 138.43 102.235) (width 0.25) (layer F.Cu) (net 9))
 (segment (start 141.4786 103.3786) (end 145.5511 103.3786) (width 0.25) (layer F.Cu) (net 9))
 (segment (start 140.335 102.235) (end 141.4786 103.3786) (width 0.25) (layer F.Cu) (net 9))
 (segment (start 138.43 102.235) (end 140.335 102.235) (width 0.25) (layer F.Cu) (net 9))
 (segment (start 139.065 100.33) (end 139.7 100.33) (width 0.25) (layer F.Cu) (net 8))
 (segment (start 139.7 100.33) (end 142.0986 102.7286) (width 0.25) (layer F.Cu) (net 8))
 (segment (start 142.0986 102.7286) (end 145.5511 102.7286) (width 0.25) (layer F.Cu) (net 8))
 (segment (start 141.605 100.33) (end 143.8025 100.33) (width 0.25) (layer F.Cu) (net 7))
 (segment (start 143.8025 100.33) (end 145.5511 102.0786) (width 0.25) (layer F.Cu) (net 7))
 (segment (start 165.78 109.665) (end 165.78 103.55) (width 0.25) (layer F.Cu) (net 20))
 (segment (start 164.3086 102.0786) (end 151.4511 102.0786) (width 0.25) (layer F.Cu) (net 20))
 (segment (start 165.78 103.55) (end 164.3086 102.0786) (width 0.25) (layer F.Cu) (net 20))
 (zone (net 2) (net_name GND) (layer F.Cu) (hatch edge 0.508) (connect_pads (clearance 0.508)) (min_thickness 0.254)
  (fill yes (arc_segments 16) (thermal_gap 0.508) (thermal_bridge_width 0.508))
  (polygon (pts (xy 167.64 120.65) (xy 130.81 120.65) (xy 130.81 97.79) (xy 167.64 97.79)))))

